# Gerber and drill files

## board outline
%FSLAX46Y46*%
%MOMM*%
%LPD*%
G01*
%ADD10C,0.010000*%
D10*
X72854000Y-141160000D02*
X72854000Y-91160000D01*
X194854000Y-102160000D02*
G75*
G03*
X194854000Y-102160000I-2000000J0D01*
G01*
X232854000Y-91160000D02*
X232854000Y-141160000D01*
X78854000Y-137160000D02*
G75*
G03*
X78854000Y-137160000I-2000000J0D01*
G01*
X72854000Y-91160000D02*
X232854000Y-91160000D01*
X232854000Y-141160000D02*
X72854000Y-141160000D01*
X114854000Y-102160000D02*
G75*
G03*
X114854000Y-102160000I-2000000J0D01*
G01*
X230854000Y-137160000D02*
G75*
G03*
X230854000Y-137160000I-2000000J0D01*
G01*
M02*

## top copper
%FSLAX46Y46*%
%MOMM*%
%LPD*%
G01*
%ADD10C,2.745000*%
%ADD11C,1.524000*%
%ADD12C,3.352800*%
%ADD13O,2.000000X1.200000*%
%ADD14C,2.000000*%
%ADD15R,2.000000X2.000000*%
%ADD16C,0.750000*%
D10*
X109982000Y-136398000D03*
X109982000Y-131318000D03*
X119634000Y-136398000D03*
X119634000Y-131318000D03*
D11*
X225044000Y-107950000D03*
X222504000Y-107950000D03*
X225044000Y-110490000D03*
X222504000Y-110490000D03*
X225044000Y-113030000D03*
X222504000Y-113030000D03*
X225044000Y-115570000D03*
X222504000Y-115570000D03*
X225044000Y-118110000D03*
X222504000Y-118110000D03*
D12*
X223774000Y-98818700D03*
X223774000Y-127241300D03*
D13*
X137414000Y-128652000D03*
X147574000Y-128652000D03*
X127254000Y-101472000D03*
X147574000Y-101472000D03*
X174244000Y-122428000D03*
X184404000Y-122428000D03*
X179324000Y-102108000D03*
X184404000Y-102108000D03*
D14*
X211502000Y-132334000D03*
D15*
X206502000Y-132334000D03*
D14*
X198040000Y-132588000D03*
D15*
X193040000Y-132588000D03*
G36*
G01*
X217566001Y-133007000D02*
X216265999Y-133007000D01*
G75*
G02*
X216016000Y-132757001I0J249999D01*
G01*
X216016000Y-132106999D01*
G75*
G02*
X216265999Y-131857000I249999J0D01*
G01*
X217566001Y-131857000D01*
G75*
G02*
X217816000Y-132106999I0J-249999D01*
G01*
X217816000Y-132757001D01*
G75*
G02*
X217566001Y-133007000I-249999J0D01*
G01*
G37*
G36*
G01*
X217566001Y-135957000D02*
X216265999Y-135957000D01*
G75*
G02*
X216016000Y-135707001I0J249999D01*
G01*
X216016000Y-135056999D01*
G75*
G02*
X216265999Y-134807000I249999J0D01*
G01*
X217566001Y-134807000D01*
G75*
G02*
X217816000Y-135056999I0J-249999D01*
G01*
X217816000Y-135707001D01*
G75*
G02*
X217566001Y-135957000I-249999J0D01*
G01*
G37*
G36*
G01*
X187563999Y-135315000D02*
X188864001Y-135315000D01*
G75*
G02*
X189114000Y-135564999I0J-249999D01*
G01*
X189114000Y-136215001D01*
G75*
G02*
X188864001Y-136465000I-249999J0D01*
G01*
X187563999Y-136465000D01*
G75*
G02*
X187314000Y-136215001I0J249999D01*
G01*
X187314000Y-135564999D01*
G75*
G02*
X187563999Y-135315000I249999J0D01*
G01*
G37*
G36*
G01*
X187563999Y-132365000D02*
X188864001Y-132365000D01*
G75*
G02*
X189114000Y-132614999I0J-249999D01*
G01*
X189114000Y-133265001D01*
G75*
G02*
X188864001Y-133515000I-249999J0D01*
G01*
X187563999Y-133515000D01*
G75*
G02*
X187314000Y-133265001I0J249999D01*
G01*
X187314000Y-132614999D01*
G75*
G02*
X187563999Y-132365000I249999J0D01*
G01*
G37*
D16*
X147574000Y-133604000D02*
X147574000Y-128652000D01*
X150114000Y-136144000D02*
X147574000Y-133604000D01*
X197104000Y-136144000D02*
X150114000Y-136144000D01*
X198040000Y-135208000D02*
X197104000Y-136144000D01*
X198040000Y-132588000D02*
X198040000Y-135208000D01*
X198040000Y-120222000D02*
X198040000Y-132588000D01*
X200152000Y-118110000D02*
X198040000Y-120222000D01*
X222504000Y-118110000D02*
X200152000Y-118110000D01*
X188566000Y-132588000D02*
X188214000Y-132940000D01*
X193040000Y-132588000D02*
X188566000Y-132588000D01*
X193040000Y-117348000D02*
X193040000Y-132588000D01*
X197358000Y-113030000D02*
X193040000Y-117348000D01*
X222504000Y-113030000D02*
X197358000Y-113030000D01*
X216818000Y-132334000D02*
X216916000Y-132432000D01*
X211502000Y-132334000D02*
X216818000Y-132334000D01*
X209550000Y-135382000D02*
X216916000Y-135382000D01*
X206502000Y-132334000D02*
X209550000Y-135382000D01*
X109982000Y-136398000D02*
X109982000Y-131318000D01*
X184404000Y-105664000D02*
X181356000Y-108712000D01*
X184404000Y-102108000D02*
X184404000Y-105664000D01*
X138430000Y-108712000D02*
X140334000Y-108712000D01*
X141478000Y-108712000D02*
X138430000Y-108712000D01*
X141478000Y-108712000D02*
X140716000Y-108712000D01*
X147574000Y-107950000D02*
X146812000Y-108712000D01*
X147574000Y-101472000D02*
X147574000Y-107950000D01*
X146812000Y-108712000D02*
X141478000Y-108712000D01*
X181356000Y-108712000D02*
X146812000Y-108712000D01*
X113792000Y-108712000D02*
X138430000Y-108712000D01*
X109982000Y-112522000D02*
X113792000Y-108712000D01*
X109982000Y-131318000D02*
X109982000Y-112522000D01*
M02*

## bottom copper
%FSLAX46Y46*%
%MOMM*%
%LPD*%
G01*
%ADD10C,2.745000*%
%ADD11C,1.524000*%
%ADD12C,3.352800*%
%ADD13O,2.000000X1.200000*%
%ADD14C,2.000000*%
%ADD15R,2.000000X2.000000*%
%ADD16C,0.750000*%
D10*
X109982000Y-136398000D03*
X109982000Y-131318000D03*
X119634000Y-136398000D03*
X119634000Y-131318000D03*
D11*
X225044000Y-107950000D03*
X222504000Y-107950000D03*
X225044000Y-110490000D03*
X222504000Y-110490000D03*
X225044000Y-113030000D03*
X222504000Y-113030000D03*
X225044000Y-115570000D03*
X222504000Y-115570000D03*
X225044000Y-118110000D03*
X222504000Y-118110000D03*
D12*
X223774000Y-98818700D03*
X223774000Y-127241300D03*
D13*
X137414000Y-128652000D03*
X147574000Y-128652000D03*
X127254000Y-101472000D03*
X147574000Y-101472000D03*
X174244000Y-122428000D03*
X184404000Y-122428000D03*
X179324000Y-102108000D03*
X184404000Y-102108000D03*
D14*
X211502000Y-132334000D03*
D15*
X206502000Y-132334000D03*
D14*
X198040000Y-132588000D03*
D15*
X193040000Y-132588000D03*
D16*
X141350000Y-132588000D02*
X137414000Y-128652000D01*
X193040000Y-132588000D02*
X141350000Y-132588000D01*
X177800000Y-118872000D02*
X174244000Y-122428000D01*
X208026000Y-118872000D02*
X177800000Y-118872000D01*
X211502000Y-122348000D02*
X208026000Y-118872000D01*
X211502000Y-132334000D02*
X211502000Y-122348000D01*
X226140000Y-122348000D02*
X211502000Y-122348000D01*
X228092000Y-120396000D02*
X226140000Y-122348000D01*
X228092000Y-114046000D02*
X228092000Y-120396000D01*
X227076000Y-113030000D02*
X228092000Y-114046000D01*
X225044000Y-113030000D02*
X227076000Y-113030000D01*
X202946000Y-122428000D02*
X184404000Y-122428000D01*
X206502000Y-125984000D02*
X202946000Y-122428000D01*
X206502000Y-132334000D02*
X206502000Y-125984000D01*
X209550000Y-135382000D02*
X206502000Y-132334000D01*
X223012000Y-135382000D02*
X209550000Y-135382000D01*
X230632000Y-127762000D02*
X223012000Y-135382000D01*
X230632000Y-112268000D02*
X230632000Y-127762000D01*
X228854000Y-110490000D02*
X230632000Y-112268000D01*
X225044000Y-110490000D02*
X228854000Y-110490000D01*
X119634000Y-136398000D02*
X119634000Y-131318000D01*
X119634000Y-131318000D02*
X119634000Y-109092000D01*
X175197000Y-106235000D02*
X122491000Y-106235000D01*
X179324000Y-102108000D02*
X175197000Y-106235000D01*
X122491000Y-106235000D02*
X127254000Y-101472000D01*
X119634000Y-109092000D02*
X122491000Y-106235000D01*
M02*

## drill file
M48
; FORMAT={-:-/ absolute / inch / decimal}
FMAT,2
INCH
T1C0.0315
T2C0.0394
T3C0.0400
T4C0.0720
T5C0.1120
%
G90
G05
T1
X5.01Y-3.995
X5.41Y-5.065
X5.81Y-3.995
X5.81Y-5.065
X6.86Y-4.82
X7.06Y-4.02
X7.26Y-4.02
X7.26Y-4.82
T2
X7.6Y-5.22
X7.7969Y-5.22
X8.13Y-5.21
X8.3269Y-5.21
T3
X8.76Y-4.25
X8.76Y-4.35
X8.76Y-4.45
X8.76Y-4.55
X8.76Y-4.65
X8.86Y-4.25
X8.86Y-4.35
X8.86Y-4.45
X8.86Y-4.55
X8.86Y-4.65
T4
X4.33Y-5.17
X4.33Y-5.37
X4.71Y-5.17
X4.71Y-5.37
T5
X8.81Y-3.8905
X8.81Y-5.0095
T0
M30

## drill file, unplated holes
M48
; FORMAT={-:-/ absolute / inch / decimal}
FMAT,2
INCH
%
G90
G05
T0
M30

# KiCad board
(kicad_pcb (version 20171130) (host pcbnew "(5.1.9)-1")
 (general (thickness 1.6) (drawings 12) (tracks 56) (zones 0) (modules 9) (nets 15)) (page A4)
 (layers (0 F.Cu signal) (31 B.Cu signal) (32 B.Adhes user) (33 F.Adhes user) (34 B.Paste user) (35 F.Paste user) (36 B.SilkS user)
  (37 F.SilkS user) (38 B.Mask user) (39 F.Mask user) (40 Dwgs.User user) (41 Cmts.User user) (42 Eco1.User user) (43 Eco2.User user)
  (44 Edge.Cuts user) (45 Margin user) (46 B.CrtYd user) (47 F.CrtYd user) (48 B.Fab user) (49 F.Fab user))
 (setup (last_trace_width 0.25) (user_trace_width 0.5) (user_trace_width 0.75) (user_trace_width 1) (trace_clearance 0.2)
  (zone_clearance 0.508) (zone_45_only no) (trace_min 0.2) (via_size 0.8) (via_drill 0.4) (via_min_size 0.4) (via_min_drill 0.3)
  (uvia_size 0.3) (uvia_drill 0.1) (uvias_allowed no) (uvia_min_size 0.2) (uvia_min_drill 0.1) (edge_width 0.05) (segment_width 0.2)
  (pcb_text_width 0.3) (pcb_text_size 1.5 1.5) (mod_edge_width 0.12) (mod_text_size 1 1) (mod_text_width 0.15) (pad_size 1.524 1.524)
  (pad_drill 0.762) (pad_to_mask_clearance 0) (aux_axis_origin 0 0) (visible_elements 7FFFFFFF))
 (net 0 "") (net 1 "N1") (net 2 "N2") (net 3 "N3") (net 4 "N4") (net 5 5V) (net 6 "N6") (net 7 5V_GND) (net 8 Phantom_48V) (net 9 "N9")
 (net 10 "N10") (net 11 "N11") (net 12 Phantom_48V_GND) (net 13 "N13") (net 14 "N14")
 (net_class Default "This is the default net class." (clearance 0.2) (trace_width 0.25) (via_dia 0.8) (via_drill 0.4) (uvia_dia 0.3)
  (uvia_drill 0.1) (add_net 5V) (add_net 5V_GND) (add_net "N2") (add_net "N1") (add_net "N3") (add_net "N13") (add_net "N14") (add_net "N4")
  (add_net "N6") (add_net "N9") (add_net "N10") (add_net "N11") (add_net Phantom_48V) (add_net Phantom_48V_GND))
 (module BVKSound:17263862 (layer F.Cu) (at 109.982 136.398 90)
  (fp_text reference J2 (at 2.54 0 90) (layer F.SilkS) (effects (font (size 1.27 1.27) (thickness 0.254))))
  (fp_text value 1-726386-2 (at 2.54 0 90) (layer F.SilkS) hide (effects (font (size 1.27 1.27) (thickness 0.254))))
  (pad 1 thru_hole circle (at 0 0 90) (size 2.745 2.745) (drill 1.83) (layers *.Cu *.Mask) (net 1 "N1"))
  (pad 2 thru_hole circle (at 5.08 0 90) (size 2.745 2.745) (drill 1.83) (layers *.Cu *.Mask) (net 1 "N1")))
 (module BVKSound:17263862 (layer F.Cu) (at 119.634 136.398 90)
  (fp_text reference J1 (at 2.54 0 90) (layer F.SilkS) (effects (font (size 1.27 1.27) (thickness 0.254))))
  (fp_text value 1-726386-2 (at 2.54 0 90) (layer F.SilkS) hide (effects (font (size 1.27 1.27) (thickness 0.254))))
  (pad 1 thru_hole circle (at 0 0 90) (size 2.745 2.745) (drill 1.83) (layers *.Cu *.Mask) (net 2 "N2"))
  (pad 2 thru_hole circle (at 5.08 0 90) (size 2.745 2.745) (drill 1.83) (layers *.Cu *.Mask) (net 2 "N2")))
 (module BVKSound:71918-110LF (layer F.Cu) (at 225.044 107.95 270)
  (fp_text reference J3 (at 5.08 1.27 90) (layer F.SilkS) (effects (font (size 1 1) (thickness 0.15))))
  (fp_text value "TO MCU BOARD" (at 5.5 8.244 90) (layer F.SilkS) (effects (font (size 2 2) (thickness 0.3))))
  (pad 1 thru_hole circle (at 0 0 270) (size 1.524 1.524) (drill 1.016) (layers *.Cu *.Mask) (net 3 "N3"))
  (pad 2 thru_hole circle (at 0 2.54 270) (size 1.524 1.524) (drill 1.016) (layers *.Cu *.Mask) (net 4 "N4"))
  (pad 3 thru_hole circle (at 2.54 0 270) (size 1.524 1.524) (drill 1.016) (layers *.Cu *.Mask) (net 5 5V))
  (pad 4 thru_hole circle (at 2.54 2.54 270) (size 1.524 1.524) (drill 1.016) (layers *.Cu *.Mask) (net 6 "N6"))
  (pad 5 thru_hole circle (at 5.08 0 270) (size 1.524 1.524) (drill 1.016) (layers *.Cu *.Mask) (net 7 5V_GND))
  (pad 6 thru_hole circle (at 5.08 2.54 270) (size 1.524 1.524) (drill 1.016) (layers *.Cu *.Mask) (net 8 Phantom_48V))
  (pad 7 thru_hole circle (at 7.62 0 270) (size 1.524 1.524) (drill 1.016) (layers *.Cu *.Mask) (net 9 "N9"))
  (pad 8 thru_hole circle (at 7.62 2.54 270) (size 1.524 1.524) (drill 1.016) (layers *.Cu *.Mask) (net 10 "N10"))
  (pad 9 thru_hole circle (at 10.16 0 270) (size 1.524 1.524) (drill 1.016) (layers *.Cu *.Mask) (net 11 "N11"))
  (pad 10 thru_hole circle (at 10.16 2.54 270) (size 1.524 1.524) (drill 1.016) (layers *.Cu *.Mask) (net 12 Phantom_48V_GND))
  (pad 11 thru_hole circle (at -9.1313 1.27 270) (size 3.3528 3.3528) (drill 2.8448) (layers *.Cu *.Mask) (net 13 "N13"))
  (pad 12 thru_hole circle (at 19.2913 1.27 270) (size 3.3528 3.3528) (drill 2.8448) (layers *.Cu *.Mask) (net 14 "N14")))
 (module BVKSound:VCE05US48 (layer F.Cu) (at 137.414 115.062 270)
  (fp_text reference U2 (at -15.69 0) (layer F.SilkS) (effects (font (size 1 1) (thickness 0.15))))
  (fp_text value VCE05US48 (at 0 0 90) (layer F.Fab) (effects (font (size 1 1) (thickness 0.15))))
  (pad 3 thru_hole oval (at 13.59 0 270) (size 1.2 2) (drill 0.8) (layers *.Cu *.Mask) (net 8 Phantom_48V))
  (pad 4 thru_hole oval (at 13.59 -10.16 270) (size 1.2 2) (drill 0.8) (layers *.Cu *.Mask) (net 12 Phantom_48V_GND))
  (pad 1 thru_hole oval (at -13.59 10.16 270) (size 1.2 2) (drill 0.8) (layers *.Cu *.Mask) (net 2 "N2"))
  (pad 2 thru_hole oval (at -13.59 -10.16 270) (size 1.2 2) (drill 0.8) (layers *.Cu *.Mask) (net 1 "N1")))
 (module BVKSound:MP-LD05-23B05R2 (layer F.Cu) (at 174.244 112.268 270)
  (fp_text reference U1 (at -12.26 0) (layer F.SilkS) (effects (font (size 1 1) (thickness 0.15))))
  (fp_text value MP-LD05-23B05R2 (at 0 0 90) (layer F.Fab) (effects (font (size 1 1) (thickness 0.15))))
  (pad 4 thru_hole oval (at 10.16 0 270) (size 1.2 2) (drill 0.8) (layers *.Cu *.Mask) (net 7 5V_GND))
  (pad 3 thru_hole oval (at 10.16 -10.16 270) (size 1.2 2) (drill 0.8) (layers *.Cu *.Mask) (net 5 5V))
  (pad 1 thru_hole oval (at -10.16 -5.08 270) (size 1.2 2) (drill 0.8) (layers *.Cu *.Mask) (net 2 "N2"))
  (pad 2 thru_hole oval (at -10.16 -10.16 270) (size 1.2 2) (drill 0.8) (layers *.Cu *.Mask) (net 1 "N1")))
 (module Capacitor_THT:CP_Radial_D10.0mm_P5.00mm (layer F.Cu) (at 206.502 132.334)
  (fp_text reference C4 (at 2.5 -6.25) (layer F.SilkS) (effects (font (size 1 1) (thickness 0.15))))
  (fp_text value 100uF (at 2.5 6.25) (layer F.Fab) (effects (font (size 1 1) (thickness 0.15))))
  (pad 2 thru_hole circle (at 5 0) (size 2 2) (drill 1) (layers *.Cu *.Mask) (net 7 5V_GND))
  (pad 1 thru_hole rect (at 0 0) (size 2 2) (drill 1) (layers *.Cu *.Mask) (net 5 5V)))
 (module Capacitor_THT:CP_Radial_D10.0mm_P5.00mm (layer F.Cu) (at 193.04 132.588)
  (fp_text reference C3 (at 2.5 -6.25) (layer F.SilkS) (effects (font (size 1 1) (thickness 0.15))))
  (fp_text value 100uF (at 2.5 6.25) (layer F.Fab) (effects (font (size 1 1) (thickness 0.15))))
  (pad 2 thru_hole circle (at 5 0) (size 2 2) (drill 1) (layers *.Cu *.Mask) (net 12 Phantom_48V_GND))
  (pad 1 thru_hole rect (at 0 0) (size 2 2) (drill 1) (layers *.Cu *.Mask) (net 8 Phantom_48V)))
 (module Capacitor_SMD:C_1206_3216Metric (layer F.Cu) (at 216.916 133.907 90)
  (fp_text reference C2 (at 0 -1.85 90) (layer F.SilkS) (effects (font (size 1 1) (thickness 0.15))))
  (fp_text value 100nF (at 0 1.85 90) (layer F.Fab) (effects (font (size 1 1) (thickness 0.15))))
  (pad 2 smd roundrect (at 1.475 0 90) (size 1.15 1.8) (layers F.Cu F.Paste F.Mask) (roundrect_rratio 0.2173904347826087) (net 7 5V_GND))
  (pad 1 smd roundrect (at -1.475 0 90) (size 1.15 1.8) (layers F.Cu F.Paste F.Mask) (roundrect_rratio 0.2173904347826087) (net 5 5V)))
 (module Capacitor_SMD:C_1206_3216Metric (layer F.Cu) (at 188.214 134.415 270)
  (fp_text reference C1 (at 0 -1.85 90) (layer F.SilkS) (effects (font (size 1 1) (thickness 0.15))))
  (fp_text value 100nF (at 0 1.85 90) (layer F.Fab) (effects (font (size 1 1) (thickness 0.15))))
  (pad 2 smd roundrect (at 1.475 0 270) (size 1.15 1.8) (layers F.Cu F.Paste F.Mask) (roundrect_rratio 0.2173904347826087)
   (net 12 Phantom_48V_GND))
  (pad 1 smd roundrect (at -1.475 0 270) (size 1.15 1.8) (layers F.Cu F.Paste F.Mask) (roundrect_rratio 0.2173904347826087)
   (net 8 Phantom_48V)))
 (gr_line (start 72.854 141.16) (end 72.854 91.16) (layer Edge.Cuts) (width 0.01))
 (gr_circle (center 192.854 102.16) (end 194.854 102.16) (layer Edge.Cuts) (width 0.01))
 (gr_line (start 232.854 91.16) (end 232.854 141.16) (layer Edge.Cuts) (width 0.01))
 (gr_circle (center 76.854 137.16) (end 78.854 137.16) (layer Edge.Cuts) (width 0.01))
 (gr_line (start 72.854 91.16) (end 232.854 91.16) (layer Edge.Cuts) (width 0.01))
 (gr_line (start 232.854 141.16) (end 72.854 141.16) (layer Edge.Cuts) (width 0.01))
 (gr_circle (center 112.854 102.16) (end 114.854 102.16) (layer Edge.Cuts) (width 0.01))
 (gr_circle (center 228.854 137.16) (end 230.854 137.16) (layer Edge.Cuts) (width 0.01))
 (segment (start 147.574 133.604) (end 147.574 128.652) (width 0.75) (layer F.Cu) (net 12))
 (segment (start 150.114 136.144) (end 147.574 133.604) (width 0.75) (layer F.Cu) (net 12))
 (segment (start 197.104 136.144) (end 150.114 136.144) (width 0.75) (layer F.Cu) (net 12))
 (segment (start 198.04 135.208) (end 197.104 136.144) (width 0.75) (layer F.Cu) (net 12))
 (segment (start 198.04 132.588) (end 198.04 135.208) (width 0.75) (layer F.Cu) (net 12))
 (segment (start 198.04 120.222) (end 198.04 132.588) (width 0.75) (layer F.Cu) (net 12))
 (segment (start 200.152 118.11) (end 198.04 120.222) (width 0.75) (layer F.Cu) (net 12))
 (segment (start 222.504 118.11) (end 200.152 118.11) (width 0.75) (layer F.Cu) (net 12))
 (segment (start 141.35 132.588) (end 137.414 128.652) (width 0.75) (layer B.Cu) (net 8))
 (segment (start 193.04 132.588) (end 141.35 132.588) (width 0.75) (layer B.Cu) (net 8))
 (segment (start 188.566 132.588) (end 188.214 132.94) (width 0.75) (layer F.Cu) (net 8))
 (segment (start 193.04 132.588) (end 188.566 132.588) (width 0.75) (layer F.Cu) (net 8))
 (segment (start 193.04 117.348) (end 193.04 132.588) (width 0.75) (layer F.Cu) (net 8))
 (segment (start 197.358 113.03) (end 193.04 117.348) (width 0.75) (layer F.Cu) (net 8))
 (segment (start 222.504 113.03) (end 197.358 113.03) (width 0.75) (layer F.Cu) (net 8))
 (segment (start 216.818 132.334) (end 216.916 132.432) (width 0.75) (layer F.Cu) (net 7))
 (segment (start 211.502 132.334) (end 216.818 132.334) (width 0.75) (layer F.Cu) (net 7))
 (segment (start 177.8 118.872) (end 174.244 122.428) (width 0.75) (layer B.Cu) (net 7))
 (segment (start 208.026 118.872) (end 177.8 118.872) (width 0.75) (layer B.Cu) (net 7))
 (segment (start 211.502 122.348) (end 208.026 118.872) (width 0.75) (layer B.Cu) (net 7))
 (segment (start 211.502 132.334) (end 211.502 122.348) (width 0.75) (layer B.Cu) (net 7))
 (segment (start 226.14 122.348) (end 211.502 122.348) (width 0.75) (layer B.Cu) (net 7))
 (segment (start 228.092 120.396) (end 226.14 122.348) (width 0.75) (layer B.Cu) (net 7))
 (segment (start 228.092 114.046) (end 228.092 120.396) (width 0.75) (layer B.Cu) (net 7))
 (segment (start 227.076 113.03) (end 228.092 114.046) (width 0.75) (layer B.Cu) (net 7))
 (segment (start 225.044 113.03) (end 227.076 113.03) (width 0.75) (layer B.Cu) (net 7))
 (segment (start 209.55 135.382) (end 216.916 135.382) (width 0.75) (layer F.Cu) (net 5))
 (segment (start 206.502 132.334) (end 209.55 135.382) (width 0.75) (layer F.Cu) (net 5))
 (segment (start 202.946 122.428) (end 184.404 122.428) (width 0.75) (layer B.Cu) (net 5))
 (segment (start 206.502 125.984) (end 202.946 122.428) (width 0.75) (layer B.Cu) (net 5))
 (segment (start 206.502 132.334) (end 206.502 125.984) (width 0.75) (layer B.Cu) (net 5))
 (segment (start 209.55 135.382) (end 206.502 132.334) (width 0.75) (layer B.Cu) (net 5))
 (segment (start 223.012 135.382) (end 209.55 135.382) (width 0.75) (layer B.Cu) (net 5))
 (segment (start 230.632 127.762) (end 223.012 135.382) (width 0.75) (layer B.Cu) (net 5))
 (segment (start 230.632 112.268) (end 230.632 127.762) (width 0.75) (layer B.Cu) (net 5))
 (segment (start 228.854 110.49) (end 230.632 112.268) (width 0.75) (layer B.Cu) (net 5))
 (segment (start 225.044 110.49) (end 228.854 110.49) (width 0.75) (layer B.Cu) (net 5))
 (segment (start 119.634 136.398) (end 119.634 131.318) (width 0.75) (layer B.Cu) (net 2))
 (segment (start 119.634 131.318) (end 119.634 109.092) (width 0.75) (layer B.Cu) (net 2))
 (segment (start 175.197 106.235) (end 122.491 106.235) (width 0.75) (layer B.Cu) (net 2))
 (segment (start 179.324 102.108) (end 175.197 106.235) (width 0.75) (layer B.Cu) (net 2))
 (segment (start 122.491 106.235) (end 127.254 101.472) (width 0.75) (layer B.Cu) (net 2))
 (segment (start 119.634 109.092) (end 122.491 106.235) (width 0.75) (layer B.Cu) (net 2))
 (segment (start 109.982 136.398) (end 109.982 131.318) (width 0.75) (layer F.Cu) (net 1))
 (segment (start 184.404 105.664) (end 181.356 108.712) (width 0.75) (layer F.Cu) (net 1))
 (segment (start 184.404 102.108) (end 184.404 105.664) (width 0.75) (layer F.Cu) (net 1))
 (segment (start 138.43 108.712) (end 140.334 108.712) (width 0.75) (layer F.Cu) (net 1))
 (segment (start 141.478 108.712) (end 138.43 108.712) (width 0.75) (layer F.Cu) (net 1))
 (segment (start 141.478 108.712) (end 140.716 108.712) (width 0.75) (layer F.Cu) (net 1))
 (segment (start 147.574 107.95) (end 146.812 108.712) (width 0.75) (layer F.Cu) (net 1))
 (segment (start 147.574 101.472) (end 147.574 107.95) (width 0.75) (layer F.Cu) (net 1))
 (segment (start 146.812 108.712) (end 141.478 108.712) (width 0.75) (layer F.Cu) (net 1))
 (segment (start 181.356 108.712) (end 146.812 108.712) (width 0.75) (layer F.Cu) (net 1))
 (segment (start 113.792 108.712) (end 138.43 108.712) (width 0.75) (layer F.Cu) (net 1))
 (segment (start 109.982 112.522) (end 113.792 108.712) (width 0.75) (layer F.Cu) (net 1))
 (segment (start 109.982 131.318) (end 109.982 112.522) (width 0.75) (layer F.Cu) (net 1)))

